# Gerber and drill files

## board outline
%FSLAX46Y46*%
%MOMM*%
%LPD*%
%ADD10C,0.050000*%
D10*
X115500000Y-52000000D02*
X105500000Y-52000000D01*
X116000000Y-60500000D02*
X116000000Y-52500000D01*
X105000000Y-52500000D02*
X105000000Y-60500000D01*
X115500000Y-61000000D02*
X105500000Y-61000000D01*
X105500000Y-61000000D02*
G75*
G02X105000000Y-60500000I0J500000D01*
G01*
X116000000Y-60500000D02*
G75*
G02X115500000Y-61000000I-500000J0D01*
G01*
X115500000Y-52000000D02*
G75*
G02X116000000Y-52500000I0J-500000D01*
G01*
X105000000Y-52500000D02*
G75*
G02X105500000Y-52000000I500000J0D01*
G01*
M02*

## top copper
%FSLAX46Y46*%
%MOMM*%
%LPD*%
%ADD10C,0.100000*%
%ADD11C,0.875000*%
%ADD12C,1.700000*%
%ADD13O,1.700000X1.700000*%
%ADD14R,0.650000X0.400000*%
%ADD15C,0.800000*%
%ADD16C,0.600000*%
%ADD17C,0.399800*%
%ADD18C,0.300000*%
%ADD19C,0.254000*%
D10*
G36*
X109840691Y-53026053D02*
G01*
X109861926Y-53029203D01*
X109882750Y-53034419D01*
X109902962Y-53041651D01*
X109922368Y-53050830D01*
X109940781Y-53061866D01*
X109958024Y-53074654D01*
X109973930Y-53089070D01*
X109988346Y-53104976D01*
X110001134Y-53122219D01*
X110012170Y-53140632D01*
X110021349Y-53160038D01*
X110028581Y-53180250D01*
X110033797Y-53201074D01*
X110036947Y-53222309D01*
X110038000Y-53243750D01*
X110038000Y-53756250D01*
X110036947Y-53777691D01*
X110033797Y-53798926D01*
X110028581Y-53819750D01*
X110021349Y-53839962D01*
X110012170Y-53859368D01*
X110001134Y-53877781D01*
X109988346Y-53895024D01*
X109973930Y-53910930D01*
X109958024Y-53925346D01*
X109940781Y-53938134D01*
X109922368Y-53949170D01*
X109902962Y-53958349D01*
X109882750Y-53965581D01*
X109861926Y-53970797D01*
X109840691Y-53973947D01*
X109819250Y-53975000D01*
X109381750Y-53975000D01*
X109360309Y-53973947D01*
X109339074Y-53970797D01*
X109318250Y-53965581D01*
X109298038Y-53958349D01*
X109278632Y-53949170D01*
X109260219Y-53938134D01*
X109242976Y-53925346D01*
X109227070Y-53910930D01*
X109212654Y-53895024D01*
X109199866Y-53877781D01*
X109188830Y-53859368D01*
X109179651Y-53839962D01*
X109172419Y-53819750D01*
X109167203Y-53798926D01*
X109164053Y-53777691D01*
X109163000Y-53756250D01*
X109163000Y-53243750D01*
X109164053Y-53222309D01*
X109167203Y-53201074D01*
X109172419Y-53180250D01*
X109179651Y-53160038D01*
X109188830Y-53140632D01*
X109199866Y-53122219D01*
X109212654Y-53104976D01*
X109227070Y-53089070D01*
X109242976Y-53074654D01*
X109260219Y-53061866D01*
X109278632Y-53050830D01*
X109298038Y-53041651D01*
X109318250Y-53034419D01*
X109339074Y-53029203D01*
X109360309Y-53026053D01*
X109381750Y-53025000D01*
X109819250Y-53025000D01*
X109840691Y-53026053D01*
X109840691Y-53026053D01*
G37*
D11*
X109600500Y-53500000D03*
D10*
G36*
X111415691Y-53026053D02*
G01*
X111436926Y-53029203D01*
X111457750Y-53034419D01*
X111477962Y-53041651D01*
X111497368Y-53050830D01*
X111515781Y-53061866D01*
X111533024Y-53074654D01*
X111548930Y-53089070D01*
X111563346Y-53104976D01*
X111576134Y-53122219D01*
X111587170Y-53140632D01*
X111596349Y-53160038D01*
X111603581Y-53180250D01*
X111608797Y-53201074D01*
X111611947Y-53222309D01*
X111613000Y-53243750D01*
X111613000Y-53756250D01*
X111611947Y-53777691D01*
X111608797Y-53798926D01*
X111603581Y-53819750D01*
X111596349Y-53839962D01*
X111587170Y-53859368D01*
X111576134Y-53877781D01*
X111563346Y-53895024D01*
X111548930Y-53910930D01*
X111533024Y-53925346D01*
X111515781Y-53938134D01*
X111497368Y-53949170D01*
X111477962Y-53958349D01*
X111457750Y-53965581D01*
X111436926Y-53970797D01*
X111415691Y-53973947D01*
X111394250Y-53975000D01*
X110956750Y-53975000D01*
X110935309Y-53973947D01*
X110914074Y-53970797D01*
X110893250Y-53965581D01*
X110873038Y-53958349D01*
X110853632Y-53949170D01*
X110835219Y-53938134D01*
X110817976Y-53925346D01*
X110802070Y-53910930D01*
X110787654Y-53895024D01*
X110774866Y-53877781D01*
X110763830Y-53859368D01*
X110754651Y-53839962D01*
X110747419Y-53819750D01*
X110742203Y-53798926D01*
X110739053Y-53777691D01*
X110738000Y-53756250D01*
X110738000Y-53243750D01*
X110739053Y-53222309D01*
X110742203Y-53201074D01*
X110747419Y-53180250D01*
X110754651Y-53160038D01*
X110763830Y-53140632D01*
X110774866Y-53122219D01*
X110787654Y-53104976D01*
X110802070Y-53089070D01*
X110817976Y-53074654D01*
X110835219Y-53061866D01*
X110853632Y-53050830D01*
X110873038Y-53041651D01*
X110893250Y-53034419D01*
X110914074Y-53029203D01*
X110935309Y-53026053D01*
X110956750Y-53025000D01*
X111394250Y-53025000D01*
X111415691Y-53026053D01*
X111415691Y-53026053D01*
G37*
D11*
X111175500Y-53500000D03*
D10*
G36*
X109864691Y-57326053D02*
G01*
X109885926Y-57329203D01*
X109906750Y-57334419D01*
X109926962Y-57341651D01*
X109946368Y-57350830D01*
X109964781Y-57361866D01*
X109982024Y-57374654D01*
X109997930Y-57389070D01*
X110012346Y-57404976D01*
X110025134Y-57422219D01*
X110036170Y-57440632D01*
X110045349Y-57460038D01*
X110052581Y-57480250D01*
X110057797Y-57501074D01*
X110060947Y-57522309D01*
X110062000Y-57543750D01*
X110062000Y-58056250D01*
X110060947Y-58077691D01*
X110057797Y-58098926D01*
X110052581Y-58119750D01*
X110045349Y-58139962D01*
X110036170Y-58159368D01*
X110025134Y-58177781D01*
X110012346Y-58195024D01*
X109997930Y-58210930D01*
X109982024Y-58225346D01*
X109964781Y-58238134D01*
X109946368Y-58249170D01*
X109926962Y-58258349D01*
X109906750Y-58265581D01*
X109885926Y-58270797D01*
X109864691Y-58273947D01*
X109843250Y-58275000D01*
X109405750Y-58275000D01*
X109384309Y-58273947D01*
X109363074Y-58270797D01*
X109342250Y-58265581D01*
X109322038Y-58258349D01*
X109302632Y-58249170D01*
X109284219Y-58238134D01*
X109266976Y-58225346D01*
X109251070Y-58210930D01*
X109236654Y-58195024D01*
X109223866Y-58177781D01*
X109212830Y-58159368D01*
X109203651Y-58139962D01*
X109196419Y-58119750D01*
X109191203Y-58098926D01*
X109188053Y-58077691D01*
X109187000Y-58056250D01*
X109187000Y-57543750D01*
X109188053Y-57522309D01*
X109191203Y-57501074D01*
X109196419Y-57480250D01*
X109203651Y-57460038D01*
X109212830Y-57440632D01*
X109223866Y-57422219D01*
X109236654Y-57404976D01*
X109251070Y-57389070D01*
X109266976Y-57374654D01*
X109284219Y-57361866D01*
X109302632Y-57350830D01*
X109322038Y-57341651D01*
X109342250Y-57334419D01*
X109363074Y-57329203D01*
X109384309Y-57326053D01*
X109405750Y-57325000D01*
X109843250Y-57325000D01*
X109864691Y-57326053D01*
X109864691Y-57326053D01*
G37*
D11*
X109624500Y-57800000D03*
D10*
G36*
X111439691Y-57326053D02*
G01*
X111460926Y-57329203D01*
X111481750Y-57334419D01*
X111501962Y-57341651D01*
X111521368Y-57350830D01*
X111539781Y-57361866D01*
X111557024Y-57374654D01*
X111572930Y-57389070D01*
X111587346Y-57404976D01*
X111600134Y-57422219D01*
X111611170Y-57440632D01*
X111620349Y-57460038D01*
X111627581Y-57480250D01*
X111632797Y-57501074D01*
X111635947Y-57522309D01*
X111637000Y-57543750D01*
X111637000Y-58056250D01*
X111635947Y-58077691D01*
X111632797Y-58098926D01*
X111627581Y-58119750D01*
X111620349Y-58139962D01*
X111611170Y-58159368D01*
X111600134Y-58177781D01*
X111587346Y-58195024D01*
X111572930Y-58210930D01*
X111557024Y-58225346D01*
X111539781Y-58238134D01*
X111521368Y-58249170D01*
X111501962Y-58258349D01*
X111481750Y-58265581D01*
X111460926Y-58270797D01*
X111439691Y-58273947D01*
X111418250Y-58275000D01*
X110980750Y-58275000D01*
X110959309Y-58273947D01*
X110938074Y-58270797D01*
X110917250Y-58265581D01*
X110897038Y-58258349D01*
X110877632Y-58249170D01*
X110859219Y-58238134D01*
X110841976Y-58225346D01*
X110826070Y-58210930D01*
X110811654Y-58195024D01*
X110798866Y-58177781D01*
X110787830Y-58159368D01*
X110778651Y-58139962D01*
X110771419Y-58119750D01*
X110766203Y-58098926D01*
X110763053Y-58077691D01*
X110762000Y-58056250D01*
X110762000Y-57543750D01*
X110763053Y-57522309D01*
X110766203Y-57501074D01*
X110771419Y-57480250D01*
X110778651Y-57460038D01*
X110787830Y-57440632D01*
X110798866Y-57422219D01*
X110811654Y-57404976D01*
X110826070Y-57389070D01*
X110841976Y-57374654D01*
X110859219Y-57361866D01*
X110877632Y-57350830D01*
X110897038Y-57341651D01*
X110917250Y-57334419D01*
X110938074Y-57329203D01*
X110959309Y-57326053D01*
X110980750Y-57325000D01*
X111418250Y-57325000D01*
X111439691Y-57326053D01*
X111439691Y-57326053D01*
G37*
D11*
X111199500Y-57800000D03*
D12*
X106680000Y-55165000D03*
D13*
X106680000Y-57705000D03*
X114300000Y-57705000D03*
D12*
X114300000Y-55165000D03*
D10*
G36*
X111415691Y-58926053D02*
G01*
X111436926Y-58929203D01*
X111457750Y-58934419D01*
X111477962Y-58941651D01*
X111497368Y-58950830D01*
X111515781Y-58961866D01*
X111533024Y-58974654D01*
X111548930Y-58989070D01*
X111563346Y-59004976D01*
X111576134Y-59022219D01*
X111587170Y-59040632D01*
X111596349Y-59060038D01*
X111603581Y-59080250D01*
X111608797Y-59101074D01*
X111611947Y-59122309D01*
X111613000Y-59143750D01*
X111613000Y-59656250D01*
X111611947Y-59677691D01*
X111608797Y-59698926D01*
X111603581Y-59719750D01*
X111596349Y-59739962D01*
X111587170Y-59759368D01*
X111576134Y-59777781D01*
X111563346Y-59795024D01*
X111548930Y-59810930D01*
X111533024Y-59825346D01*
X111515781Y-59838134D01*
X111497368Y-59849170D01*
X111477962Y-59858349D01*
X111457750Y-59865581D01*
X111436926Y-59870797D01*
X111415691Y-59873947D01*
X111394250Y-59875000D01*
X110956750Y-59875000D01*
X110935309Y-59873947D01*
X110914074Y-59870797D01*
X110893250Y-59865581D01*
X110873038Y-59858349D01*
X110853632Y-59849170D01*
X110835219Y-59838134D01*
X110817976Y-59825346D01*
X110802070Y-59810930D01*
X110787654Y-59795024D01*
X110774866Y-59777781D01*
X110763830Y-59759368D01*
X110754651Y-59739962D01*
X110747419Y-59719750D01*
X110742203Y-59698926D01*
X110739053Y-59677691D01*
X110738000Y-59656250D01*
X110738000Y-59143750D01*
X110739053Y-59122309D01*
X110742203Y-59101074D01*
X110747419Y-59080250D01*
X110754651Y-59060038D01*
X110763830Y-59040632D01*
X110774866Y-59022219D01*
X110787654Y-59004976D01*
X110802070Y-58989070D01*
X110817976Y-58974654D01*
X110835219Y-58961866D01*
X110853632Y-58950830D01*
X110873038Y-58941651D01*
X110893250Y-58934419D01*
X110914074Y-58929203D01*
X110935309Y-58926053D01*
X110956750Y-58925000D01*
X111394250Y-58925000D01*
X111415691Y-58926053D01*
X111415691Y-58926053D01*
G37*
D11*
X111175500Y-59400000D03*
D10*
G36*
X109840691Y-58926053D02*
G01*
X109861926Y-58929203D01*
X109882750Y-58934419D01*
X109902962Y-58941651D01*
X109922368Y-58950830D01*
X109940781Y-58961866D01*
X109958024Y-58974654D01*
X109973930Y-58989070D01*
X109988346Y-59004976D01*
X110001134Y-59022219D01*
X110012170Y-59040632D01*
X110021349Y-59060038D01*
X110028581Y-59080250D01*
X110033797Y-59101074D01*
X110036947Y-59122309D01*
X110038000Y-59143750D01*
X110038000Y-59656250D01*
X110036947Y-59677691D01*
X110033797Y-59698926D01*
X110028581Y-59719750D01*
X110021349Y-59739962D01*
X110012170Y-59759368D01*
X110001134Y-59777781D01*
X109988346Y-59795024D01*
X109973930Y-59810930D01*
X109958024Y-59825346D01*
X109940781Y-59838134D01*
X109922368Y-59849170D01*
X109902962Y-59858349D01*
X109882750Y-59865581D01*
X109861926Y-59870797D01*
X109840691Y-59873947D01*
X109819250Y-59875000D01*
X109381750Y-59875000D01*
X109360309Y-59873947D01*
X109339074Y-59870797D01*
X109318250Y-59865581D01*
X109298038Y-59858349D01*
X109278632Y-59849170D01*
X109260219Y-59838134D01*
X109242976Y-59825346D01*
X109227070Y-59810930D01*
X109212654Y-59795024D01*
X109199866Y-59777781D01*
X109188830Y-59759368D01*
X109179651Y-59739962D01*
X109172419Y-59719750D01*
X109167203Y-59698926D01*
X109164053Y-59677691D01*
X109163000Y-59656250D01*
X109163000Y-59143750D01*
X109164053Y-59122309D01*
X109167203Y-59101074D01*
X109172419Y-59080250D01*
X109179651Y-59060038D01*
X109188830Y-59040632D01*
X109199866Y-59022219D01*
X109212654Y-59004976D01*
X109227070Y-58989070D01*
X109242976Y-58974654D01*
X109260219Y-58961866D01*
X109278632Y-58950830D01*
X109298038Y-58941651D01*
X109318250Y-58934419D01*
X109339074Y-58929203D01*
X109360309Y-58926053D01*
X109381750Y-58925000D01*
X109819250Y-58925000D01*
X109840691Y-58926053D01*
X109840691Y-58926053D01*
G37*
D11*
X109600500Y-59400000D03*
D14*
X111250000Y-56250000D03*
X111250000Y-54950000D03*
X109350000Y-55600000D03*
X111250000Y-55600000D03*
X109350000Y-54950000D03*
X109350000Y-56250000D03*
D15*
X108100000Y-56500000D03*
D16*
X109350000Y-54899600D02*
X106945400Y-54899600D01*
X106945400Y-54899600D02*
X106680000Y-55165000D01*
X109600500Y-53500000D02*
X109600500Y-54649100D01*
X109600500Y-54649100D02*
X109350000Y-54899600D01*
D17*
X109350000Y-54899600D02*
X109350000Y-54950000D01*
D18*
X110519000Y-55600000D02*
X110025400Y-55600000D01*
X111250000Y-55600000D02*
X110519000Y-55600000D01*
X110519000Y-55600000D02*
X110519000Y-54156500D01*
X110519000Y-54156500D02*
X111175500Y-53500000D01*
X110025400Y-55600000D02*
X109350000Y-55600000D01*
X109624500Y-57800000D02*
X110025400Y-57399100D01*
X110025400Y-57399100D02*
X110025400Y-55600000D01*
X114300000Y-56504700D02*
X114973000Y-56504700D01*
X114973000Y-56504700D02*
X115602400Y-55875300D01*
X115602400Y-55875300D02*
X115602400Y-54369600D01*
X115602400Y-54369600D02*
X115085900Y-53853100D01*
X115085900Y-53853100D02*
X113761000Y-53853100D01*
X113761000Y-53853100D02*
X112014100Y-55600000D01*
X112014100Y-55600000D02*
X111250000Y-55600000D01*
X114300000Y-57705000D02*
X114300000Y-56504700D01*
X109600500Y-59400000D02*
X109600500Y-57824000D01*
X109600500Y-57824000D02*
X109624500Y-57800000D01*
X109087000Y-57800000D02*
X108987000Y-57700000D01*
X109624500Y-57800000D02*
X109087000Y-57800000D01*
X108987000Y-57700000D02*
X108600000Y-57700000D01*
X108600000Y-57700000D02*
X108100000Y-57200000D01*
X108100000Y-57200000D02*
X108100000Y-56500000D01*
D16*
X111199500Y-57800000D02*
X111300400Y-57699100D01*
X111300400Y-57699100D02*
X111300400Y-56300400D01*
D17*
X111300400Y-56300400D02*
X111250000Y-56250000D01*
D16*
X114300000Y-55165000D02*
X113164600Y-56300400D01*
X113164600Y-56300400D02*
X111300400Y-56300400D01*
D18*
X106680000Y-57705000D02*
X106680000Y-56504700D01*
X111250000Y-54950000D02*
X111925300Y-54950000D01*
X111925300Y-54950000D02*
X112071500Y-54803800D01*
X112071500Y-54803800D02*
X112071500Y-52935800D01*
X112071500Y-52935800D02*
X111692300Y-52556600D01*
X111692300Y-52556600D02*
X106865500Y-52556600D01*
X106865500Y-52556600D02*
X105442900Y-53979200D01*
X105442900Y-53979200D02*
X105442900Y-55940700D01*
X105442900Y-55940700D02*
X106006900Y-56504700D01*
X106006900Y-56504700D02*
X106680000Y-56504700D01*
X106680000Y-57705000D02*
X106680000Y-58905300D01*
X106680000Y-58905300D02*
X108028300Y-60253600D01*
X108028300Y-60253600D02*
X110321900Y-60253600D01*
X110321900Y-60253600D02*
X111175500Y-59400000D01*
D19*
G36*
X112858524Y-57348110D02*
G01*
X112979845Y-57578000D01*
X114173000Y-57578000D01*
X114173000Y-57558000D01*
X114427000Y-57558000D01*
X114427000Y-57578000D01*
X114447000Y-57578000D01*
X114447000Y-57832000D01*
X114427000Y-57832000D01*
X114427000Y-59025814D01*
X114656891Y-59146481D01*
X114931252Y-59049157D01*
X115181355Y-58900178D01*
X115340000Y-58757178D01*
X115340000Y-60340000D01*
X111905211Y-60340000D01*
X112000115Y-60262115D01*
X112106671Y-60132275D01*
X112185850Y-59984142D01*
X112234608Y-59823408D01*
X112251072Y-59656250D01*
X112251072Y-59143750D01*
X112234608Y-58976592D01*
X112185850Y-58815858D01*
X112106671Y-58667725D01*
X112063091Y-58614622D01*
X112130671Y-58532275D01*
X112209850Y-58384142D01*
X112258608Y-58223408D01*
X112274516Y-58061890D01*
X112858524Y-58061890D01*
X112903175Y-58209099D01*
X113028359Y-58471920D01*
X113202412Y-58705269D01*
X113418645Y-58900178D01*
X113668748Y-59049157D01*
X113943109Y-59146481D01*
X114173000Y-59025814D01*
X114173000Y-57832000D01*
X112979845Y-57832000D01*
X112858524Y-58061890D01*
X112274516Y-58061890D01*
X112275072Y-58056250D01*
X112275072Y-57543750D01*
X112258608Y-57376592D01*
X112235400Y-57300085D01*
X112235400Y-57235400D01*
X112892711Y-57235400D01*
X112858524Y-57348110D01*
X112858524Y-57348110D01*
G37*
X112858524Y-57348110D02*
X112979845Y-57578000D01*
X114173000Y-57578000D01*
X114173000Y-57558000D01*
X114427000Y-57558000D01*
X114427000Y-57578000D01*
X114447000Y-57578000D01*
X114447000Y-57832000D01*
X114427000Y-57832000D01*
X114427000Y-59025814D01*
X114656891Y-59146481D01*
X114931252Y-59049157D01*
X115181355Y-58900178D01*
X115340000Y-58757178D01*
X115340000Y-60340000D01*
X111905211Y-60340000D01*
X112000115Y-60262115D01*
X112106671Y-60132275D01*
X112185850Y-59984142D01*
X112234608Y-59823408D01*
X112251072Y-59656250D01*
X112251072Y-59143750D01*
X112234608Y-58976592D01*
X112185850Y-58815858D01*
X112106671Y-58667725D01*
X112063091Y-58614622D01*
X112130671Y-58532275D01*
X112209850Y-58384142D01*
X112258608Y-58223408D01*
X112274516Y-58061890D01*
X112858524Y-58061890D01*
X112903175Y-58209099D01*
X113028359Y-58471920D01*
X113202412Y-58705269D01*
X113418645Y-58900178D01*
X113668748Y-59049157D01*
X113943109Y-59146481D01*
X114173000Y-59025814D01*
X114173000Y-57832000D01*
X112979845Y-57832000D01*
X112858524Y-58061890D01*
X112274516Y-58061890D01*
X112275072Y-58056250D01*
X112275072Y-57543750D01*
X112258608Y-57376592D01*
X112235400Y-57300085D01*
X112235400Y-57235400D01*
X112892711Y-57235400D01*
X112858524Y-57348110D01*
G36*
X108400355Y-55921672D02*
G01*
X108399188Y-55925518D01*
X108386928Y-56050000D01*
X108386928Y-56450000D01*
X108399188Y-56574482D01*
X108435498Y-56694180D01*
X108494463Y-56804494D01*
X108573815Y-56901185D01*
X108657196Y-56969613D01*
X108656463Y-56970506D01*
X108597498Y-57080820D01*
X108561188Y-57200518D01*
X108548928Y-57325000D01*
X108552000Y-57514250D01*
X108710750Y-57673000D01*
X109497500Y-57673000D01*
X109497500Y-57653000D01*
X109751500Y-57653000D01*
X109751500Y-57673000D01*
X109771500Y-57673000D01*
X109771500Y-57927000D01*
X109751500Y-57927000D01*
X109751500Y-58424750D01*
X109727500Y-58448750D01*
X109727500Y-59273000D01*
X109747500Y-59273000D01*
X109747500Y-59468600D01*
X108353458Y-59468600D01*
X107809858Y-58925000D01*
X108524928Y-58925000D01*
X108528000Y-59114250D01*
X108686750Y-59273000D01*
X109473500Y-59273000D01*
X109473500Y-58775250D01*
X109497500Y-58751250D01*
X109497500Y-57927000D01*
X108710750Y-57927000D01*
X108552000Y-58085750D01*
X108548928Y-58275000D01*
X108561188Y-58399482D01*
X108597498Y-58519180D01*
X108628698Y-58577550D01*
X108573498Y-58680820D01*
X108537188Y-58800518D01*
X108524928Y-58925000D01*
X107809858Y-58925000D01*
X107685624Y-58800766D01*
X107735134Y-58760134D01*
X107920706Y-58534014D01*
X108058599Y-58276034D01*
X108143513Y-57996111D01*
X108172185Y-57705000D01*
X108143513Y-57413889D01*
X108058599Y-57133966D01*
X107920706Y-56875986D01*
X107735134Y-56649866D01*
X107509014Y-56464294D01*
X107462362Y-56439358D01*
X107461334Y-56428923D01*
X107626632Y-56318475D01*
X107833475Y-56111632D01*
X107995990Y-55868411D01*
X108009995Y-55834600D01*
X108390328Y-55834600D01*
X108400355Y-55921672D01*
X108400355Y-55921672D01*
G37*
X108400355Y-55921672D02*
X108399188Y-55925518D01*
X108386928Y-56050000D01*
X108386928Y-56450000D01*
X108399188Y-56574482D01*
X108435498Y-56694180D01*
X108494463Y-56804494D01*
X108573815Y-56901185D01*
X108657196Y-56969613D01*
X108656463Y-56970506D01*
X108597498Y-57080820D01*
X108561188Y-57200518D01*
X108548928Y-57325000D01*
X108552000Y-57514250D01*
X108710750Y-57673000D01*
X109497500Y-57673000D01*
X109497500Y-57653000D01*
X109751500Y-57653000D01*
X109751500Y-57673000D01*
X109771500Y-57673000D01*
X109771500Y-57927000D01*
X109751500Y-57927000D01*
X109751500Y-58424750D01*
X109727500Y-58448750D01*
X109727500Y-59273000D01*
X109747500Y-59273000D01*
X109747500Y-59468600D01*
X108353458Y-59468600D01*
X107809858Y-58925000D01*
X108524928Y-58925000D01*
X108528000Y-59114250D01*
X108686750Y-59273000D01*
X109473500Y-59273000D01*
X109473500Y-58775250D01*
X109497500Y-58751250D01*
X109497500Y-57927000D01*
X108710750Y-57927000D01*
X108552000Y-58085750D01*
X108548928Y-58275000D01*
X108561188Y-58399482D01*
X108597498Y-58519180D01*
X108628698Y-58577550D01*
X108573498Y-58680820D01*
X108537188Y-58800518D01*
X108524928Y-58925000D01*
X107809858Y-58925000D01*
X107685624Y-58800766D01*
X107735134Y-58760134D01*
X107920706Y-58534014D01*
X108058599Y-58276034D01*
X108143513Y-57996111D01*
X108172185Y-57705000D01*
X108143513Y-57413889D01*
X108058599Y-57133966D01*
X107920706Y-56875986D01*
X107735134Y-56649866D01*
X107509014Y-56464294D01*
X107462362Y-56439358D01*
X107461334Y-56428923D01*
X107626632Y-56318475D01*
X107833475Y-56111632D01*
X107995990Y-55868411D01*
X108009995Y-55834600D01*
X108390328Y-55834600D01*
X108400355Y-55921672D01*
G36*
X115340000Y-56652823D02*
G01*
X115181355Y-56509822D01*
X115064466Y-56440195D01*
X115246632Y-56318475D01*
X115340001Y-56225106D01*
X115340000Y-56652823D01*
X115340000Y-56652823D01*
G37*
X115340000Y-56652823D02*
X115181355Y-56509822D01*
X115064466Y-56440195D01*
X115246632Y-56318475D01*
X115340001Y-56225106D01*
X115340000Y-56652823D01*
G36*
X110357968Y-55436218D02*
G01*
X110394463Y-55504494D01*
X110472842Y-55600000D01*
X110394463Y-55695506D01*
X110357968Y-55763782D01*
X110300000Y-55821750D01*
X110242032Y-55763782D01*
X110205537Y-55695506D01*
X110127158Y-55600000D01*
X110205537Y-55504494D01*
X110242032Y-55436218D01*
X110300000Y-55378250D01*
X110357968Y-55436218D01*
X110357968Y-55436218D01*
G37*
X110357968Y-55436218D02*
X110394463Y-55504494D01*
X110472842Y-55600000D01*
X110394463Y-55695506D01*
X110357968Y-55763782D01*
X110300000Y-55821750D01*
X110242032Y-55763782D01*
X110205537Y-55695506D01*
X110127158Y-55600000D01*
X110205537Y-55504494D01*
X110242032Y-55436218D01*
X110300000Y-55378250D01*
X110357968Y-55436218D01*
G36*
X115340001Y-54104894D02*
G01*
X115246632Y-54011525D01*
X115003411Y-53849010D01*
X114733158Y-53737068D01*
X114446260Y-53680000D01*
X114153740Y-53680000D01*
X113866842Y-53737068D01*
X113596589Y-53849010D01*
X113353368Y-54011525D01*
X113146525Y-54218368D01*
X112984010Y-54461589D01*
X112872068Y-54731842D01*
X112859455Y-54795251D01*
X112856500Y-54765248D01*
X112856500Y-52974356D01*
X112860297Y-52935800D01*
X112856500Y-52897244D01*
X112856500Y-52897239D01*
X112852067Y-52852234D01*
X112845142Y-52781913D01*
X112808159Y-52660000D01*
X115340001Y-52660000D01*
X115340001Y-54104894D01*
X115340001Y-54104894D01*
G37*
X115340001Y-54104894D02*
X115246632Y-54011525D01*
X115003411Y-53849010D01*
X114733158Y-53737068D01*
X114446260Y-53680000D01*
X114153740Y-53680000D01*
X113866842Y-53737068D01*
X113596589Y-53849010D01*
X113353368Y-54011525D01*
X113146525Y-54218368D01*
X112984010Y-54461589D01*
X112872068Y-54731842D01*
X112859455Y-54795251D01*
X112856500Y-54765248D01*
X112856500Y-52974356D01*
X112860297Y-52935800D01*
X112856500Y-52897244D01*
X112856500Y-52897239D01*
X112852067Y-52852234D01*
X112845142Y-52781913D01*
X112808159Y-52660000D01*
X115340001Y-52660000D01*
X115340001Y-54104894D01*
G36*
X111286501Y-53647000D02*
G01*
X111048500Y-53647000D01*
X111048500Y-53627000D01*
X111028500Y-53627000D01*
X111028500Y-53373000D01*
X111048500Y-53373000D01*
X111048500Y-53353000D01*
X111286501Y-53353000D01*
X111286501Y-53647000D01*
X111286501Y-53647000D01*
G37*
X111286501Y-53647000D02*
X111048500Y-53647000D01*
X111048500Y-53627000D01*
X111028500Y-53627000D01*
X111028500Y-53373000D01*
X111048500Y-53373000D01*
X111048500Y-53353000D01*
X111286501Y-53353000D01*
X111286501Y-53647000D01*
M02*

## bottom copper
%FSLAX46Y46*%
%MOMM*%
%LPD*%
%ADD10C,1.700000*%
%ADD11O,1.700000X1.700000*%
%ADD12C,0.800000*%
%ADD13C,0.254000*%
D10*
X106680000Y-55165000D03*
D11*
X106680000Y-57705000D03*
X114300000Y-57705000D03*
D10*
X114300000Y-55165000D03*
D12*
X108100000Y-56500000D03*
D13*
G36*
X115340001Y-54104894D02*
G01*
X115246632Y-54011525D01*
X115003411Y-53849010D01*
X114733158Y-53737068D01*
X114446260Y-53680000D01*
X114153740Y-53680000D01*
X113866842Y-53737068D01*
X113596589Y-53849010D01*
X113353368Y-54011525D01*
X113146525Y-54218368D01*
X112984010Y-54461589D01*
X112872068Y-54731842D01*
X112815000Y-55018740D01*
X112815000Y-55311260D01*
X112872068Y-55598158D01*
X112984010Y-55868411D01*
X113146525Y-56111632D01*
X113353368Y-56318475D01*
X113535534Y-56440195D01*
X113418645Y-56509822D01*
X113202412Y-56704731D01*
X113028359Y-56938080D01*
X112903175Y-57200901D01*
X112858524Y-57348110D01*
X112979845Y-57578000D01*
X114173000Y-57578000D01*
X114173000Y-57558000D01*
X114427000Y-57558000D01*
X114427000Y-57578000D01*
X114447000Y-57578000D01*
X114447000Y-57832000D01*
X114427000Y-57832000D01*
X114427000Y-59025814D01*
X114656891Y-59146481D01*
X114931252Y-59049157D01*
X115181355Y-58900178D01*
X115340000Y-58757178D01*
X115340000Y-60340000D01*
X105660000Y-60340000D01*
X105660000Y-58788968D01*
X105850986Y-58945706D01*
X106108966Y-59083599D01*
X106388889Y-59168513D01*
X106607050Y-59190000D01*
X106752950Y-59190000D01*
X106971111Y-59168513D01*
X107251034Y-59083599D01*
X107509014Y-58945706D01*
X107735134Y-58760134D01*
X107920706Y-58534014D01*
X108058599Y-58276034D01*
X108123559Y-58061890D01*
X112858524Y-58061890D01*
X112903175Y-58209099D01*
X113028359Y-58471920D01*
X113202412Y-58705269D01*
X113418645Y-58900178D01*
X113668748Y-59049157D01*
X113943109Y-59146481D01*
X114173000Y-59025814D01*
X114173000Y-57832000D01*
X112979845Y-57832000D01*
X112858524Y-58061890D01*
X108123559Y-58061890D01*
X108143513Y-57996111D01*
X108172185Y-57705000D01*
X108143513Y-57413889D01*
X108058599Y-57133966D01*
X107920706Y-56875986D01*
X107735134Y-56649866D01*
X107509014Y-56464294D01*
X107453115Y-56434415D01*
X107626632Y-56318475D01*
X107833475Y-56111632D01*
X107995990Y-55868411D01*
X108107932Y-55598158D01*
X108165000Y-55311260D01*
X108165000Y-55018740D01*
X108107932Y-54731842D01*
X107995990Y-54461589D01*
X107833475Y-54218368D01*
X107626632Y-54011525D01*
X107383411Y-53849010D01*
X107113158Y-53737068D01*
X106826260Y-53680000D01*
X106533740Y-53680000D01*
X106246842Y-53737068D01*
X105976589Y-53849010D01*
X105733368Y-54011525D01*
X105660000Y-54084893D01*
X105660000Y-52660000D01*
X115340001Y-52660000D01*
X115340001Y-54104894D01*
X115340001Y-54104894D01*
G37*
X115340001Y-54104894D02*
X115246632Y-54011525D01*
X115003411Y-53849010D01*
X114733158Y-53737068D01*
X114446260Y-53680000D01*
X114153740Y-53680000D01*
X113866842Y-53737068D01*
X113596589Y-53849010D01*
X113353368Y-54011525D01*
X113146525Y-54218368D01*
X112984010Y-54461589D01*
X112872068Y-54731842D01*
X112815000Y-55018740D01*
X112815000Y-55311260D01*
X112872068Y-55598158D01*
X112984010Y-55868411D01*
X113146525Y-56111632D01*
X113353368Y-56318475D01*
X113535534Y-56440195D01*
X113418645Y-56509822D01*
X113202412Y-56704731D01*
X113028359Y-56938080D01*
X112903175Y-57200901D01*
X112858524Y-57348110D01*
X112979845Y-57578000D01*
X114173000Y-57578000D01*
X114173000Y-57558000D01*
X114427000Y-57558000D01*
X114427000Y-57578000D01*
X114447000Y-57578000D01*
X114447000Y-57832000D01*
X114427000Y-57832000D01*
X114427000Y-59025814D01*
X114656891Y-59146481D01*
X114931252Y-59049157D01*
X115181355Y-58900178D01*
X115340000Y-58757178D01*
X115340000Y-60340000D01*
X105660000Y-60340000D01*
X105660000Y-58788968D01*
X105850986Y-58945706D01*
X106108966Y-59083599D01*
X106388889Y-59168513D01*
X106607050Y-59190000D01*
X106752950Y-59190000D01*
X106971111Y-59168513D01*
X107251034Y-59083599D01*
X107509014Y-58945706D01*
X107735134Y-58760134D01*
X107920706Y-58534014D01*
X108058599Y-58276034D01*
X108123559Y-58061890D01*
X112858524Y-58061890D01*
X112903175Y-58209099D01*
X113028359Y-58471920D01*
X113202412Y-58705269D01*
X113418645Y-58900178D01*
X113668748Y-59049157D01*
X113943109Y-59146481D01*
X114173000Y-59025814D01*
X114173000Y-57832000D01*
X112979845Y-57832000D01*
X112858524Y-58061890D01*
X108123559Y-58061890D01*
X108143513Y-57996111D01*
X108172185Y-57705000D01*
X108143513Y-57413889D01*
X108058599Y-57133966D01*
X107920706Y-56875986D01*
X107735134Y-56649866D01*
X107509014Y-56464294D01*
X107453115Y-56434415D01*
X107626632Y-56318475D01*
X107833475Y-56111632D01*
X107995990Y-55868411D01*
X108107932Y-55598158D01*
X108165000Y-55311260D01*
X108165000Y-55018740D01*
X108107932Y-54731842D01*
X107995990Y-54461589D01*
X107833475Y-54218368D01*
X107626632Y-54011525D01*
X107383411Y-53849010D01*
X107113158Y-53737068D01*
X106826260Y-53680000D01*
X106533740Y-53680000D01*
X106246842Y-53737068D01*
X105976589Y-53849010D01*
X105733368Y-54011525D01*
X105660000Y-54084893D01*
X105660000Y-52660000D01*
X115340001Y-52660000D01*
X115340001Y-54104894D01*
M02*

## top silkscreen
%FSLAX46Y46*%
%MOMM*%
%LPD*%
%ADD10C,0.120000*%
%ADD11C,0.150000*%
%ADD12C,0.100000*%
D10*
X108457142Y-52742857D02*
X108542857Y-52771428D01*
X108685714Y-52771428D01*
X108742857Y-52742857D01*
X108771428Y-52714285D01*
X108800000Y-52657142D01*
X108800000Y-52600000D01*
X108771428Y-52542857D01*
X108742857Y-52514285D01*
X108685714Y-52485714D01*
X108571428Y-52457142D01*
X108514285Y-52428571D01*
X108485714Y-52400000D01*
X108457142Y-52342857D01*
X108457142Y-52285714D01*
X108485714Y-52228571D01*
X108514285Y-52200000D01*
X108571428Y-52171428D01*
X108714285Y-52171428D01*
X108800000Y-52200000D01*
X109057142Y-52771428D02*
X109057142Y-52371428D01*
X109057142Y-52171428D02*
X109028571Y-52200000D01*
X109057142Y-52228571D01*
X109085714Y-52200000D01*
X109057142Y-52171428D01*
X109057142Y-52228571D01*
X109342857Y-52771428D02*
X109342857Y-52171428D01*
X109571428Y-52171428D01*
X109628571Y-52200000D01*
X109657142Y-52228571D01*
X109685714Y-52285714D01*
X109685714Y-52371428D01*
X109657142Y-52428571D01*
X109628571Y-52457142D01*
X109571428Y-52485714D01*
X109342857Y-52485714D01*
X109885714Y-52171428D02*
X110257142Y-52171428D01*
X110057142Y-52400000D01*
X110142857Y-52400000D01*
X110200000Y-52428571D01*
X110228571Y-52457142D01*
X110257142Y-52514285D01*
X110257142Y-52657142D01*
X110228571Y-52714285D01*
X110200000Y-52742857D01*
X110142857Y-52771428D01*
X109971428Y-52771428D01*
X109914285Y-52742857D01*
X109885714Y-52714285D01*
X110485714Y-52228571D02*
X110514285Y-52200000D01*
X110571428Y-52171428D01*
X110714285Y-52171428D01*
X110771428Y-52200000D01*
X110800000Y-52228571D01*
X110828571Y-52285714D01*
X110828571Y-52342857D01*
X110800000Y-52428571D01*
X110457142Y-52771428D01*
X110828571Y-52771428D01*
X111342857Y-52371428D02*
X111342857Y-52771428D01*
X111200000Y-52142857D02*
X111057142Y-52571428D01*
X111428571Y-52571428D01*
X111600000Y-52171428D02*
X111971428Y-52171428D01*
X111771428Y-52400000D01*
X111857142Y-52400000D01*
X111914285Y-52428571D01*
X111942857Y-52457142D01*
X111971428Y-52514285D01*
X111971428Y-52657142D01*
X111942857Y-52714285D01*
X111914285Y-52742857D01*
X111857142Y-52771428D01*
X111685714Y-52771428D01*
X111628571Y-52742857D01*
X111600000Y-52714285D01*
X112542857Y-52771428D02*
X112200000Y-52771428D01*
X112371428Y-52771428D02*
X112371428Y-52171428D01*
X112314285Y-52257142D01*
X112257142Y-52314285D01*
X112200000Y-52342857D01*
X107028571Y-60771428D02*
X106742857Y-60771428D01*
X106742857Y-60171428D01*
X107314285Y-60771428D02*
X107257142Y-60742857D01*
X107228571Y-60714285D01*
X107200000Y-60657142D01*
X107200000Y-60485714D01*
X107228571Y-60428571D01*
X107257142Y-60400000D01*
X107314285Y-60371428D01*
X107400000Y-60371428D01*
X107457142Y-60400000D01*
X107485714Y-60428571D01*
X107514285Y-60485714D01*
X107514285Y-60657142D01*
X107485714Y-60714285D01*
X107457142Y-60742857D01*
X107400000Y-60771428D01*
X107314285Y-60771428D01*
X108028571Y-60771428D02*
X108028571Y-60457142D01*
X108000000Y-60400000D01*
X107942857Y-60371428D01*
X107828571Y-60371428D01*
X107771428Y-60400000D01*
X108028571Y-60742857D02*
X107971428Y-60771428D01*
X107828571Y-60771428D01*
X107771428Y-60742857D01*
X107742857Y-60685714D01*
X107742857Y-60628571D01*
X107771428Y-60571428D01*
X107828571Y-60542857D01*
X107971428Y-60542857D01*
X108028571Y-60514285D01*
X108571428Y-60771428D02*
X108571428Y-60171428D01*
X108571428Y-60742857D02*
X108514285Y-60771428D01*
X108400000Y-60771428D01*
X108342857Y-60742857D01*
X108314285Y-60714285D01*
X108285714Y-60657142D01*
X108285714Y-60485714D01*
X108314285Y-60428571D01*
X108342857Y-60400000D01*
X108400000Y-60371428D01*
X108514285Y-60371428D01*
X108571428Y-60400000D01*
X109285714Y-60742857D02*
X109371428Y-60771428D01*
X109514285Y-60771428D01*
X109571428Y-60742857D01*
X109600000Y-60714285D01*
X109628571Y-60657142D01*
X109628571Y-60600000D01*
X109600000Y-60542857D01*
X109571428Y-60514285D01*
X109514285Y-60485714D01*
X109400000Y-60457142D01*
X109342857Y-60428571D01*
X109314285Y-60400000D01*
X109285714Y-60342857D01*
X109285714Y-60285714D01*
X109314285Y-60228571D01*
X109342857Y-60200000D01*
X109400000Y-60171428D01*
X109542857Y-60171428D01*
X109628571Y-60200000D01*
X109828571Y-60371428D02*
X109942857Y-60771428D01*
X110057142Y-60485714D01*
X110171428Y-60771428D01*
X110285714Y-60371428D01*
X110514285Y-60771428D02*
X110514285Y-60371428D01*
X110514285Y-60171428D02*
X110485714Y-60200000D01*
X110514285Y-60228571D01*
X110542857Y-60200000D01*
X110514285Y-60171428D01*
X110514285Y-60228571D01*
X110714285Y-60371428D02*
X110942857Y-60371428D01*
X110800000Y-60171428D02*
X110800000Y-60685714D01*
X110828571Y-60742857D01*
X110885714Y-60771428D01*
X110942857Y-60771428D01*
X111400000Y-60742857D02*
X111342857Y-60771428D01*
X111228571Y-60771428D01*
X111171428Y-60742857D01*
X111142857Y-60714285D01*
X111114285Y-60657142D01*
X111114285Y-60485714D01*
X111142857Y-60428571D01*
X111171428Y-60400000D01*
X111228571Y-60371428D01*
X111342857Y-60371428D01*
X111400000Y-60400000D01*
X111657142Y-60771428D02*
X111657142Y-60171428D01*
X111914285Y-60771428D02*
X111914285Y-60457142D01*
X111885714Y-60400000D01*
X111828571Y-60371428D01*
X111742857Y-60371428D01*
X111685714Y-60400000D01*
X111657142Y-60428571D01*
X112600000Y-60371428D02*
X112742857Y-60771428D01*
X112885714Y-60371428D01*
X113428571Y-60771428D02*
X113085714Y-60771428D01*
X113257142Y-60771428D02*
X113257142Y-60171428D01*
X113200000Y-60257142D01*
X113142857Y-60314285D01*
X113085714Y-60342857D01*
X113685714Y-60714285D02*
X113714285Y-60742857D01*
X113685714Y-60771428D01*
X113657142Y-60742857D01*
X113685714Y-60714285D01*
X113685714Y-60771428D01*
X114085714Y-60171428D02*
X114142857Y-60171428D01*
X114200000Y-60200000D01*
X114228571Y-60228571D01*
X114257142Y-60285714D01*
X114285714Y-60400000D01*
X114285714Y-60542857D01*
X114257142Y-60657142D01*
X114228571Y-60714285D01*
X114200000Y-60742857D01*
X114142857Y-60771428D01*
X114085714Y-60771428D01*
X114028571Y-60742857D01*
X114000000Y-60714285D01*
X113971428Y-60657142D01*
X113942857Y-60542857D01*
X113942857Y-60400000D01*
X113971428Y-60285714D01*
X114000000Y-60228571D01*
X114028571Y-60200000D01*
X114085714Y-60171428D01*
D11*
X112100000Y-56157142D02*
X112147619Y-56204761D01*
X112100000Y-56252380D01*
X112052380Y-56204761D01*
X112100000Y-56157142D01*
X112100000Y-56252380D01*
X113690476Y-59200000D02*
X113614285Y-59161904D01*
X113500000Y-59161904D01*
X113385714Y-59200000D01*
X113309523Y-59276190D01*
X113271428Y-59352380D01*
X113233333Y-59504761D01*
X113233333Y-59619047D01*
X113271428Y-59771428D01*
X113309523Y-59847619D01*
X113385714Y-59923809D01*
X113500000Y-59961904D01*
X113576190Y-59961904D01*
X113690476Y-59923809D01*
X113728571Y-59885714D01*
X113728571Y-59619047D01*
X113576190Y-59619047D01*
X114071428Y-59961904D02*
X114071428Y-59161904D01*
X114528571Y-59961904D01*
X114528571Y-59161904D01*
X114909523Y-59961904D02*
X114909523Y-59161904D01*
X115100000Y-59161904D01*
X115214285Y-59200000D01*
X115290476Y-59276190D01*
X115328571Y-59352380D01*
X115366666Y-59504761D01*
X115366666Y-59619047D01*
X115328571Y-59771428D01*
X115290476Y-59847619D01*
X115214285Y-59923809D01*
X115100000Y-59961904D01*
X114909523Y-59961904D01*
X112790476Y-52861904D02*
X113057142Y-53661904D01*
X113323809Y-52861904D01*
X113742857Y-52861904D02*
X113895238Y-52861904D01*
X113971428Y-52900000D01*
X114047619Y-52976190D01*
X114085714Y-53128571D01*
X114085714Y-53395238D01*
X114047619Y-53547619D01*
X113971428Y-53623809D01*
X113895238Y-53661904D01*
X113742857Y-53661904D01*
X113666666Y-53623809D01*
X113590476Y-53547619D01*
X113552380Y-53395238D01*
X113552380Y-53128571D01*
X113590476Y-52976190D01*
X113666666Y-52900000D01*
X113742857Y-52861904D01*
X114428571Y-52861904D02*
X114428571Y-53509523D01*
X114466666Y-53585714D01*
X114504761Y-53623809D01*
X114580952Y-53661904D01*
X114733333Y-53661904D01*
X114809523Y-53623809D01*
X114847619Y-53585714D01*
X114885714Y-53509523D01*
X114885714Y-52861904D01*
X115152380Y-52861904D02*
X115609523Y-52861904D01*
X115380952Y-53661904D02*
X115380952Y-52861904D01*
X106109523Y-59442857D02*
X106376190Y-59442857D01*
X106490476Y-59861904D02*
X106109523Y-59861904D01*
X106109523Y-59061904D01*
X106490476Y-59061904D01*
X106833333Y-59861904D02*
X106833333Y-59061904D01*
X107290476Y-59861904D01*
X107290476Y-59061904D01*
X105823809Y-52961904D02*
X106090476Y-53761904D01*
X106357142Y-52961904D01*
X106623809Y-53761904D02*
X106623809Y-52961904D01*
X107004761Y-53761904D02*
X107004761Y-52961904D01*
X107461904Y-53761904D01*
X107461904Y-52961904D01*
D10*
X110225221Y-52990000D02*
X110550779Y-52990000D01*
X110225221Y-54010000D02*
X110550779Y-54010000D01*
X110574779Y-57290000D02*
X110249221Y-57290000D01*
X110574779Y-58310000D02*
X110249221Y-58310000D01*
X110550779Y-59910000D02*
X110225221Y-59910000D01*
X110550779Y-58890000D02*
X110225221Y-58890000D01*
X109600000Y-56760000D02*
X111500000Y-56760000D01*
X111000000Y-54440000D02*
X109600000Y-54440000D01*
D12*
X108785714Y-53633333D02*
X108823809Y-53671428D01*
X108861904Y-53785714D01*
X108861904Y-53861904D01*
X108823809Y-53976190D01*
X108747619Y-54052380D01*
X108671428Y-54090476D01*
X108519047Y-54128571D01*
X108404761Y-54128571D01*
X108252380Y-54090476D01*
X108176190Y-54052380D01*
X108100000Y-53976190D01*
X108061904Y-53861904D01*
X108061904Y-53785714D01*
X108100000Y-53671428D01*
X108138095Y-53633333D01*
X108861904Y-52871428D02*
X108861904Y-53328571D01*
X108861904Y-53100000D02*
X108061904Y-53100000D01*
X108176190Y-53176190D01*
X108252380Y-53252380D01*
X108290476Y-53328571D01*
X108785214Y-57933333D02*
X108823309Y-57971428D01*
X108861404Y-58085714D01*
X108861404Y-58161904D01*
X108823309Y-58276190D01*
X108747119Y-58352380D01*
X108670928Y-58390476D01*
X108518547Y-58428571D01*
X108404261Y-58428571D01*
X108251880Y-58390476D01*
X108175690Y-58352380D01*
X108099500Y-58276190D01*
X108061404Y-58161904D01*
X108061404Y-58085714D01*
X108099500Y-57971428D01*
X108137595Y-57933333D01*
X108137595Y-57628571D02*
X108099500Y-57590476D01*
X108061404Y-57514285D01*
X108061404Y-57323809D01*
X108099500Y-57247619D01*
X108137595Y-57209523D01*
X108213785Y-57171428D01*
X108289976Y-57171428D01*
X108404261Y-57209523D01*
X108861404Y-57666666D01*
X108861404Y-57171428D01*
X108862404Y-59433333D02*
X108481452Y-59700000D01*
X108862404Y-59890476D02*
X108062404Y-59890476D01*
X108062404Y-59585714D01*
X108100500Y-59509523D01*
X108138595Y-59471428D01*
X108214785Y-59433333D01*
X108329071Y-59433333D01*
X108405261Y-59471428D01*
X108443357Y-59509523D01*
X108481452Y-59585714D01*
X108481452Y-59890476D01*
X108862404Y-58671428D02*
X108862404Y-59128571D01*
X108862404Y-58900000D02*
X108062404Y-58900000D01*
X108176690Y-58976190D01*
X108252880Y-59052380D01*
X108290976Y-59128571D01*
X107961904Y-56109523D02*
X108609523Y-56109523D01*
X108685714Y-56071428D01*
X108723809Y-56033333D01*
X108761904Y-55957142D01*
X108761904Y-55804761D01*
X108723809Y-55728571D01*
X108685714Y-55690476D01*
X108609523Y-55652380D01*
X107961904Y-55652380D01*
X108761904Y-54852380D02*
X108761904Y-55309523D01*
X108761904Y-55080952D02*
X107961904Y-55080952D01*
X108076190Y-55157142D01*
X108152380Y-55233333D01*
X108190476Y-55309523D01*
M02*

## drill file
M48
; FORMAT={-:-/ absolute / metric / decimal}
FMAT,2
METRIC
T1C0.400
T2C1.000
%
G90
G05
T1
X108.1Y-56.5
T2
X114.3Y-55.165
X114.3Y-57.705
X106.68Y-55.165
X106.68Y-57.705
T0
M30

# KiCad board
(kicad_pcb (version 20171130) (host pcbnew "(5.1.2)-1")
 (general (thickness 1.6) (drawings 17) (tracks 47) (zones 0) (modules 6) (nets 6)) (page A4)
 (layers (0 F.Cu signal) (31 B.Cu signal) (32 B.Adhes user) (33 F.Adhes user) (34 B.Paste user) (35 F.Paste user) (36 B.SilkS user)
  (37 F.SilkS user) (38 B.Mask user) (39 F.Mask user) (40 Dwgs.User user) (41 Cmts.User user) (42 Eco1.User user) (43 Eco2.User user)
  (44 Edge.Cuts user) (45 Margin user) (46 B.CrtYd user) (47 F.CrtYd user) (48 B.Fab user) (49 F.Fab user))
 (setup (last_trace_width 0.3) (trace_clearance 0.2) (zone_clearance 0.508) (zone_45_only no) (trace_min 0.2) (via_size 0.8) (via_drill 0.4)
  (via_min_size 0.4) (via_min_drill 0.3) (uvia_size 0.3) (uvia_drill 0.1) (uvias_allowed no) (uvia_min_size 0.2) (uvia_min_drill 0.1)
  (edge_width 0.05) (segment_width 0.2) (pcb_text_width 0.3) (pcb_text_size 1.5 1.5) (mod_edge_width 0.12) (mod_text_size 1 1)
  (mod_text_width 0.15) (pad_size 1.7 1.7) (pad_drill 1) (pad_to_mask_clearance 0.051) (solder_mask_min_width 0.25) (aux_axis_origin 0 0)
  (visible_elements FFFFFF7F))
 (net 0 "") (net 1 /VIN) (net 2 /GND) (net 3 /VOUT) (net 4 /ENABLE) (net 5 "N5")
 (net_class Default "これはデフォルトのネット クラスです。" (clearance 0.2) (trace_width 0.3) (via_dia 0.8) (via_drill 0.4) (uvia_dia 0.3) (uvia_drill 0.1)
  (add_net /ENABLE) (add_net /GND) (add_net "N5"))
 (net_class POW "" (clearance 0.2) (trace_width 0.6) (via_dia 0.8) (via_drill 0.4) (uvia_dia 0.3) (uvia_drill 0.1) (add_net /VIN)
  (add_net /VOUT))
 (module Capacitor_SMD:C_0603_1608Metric (layer F.Cu) (at 110.388 53.5)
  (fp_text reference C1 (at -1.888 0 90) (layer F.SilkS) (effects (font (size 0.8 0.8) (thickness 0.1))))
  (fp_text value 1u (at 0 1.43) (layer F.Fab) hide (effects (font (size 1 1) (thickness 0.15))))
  (fp_line (start -0.162779 -0.51) (end 0.162779 -0.51) (layer F.SilkS) (width 0.12))
  (fp_line (start -0.162779 0.51) (end 0.162779 0.51) (layer F.SilkS) (width 0.12))
  (pad 1 smd roundrect (at -0.7875 0) (size 0.875 0.95) (layers F.Cu F.Paste F.Mask) (roundrect_rratio 0.25) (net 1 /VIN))
  (pad 2 smd roundrect (at 0.7875 0) (size 0.875 0.95) (layers F.Cu F.Paste F.Mask) (roundrect_rratio 0.25) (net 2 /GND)))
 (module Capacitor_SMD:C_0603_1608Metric (layer F.Cu) (at 110.412 57.8 180)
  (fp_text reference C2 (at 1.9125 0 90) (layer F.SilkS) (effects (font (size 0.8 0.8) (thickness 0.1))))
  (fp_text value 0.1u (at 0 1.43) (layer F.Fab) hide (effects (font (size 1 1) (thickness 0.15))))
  (fp_line (start -0.162779 0.51) (end 0.162779 0.51) (layer F.SilkS) (width 0.12))
  (fp_line (start -0.162779 -0.51) (end 0.162779 -0.51) (layer F.SilkS) (width 0.12))
  (pad 2 smd roundrect (at 0.7875 0 180) (size 0.875 0.95) (layers F.Cu F.Paste F.Mask) (roundrect_rratio 0.25) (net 2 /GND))
  (pad 1 smd roundrect (at -0.7875 0 180) (size 0.875 0.95) (layers F.Cu F.Paste F.Mask) (roundrect_rratio 0.25) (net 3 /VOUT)))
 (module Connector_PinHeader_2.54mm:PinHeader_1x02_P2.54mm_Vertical (layer B.Cu) (at 106.68 55.165 180)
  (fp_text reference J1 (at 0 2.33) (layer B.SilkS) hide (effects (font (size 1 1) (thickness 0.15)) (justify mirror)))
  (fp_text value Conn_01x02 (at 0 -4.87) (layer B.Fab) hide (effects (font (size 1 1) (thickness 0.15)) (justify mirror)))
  (pad 1 thru_hole circle (at 0 0 180) (size 1.7 1.7) (drill 1) (layers *.Cu *.Mask) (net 1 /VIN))
  (pad 2 thru_hole oval (at 0 -2.54 180) (size 1.7 1.7) (drill 1) (layers *.Cu *.Mask) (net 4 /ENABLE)))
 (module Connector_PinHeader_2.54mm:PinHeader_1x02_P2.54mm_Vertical (layer B.Cu) (at 114.3 55.165 180)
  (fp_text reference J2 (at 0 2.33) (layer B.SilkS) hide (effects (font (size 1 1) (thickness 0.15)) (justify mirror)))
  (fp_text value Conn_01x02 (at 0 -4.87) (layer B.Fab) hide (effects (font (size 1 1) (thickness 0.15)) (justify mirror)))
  (pad 2 thru_hole oval (at 0 -2.54 180) (size 1.7 1.7) (drill 1) (layers *.Cu *.Mask) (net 2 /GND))
  (pad 1 thru_hole circle (at 0 0 180) (size 1.7 1.7) (drill 1) (layers *.Cu *.Mask) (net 3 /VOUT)))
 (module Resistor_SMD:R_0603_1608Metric (layer F.Cu) (at 110.388 59.4 180)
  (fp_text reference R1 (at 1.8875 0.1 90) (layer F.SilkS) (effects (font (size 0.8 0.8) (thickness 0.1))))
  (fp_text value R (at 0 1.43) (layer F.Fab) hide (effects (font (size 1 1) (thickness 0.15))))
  (fp_line (start -0.162779 -0.51) (end 0.162779 -0.51) (layer F.SilkS) (width 0.12))
  (fp_line (start -0.162779 0.51) (end 0.162779 0.51) (layer F.SilkS) (width 0.12))
  (pad 1 smd roundrect (at -0.7875 0 180) (size 0.875 0.95) (layers F.Cu F.Paste F.Mask) (roundrect_rratio 0.25) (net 4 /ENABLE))
  (pad 2 smd roundrect (at 0.7875 0 180) (size 0.875 0.95) (layers F.Cu F.Paste F.Mask) (roundrect_rratio 0.25) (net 2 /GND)))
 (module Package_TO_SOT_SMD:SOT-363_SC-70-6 (layer F.Cu) (at 110.3 55.6 180)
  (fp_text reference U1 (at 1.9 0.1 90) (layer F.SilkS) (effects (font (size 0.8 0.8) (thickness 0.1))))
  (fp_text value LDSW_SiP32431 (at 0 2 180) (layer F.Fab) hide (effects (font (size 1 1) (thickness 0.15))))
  (fp_line (start 0.7 -1.16) (end -1.2 -1.16) (layer F.SilkS) (width 0.12))
  (fp_line (start -0.7 1.16) (end 0.7 1.16) (layer F.SilkS) (width 0.12))
  (pad 1 smd rect (at -0.95 -0.65 180) (size 0.65 0.4) (layers F.Cu F.Paste F.Mask) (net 3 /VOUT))
  (pad 3 smd rect (at -0.95 0.65 180) (size 0.65 0.4) (layers F.Cu F.Paste F.Mask) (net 4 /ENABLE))
  (pad 5 smd rect (at 0.95 0 180) (size 0.65 0.4) (layers F.Cu F.Paste F.Mask) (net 2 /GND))
  (pad 2 smd rect (at -0.95 0 180) (size 0.65 0.4) (layers F.Cu F.Paste F.Mask) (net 2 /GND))
  (pad 4 smd rect (at 0.95 0.65 180) (size 0.65 0.4) (layers F.Cu F.Paste F.Mask) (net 1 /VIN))
  (pad 6 smd rect (at 0.95 -0.65 180) (size 0.65 0.4) (layers F.Cu F.Paste F.Mask) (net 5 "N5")))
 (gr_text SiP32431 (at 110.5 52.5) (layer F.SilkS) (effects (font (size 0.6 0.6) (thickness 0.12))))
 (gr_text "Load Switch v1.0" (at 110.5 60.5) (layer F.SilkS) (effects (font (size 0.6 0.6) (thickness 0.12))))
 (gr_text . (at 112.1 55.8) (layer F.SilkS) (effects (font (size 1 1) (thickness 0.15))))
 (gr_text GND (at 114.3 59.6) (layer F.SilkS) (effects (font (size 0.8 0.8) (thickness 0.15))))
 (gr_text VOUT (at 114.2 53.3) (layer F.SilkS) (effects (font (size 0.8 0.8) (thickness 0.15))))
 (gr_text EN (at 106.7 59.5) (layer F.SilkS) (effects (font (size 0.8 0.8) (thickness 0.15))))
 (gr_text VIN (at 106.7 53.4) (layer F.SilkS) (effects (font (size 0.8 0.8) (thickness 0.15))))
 (gr_line (start 115.5 52) (end 105.5 52) (layer Edge.Cuts) (width 0.05))
 (gr_line (start 116 60.5) (end 116 52.5) (layer Edge.Cuts) (width 0.05))
 (gr_line (start 105 52.5) (end 105 60.5) (layer Edge.Cuts) (width 0.05))
 (gr_line (start 115.5 61) (end 105.5 61) (layer Edge.Cuts) (width 0.05))
 (gr_arc (start 105.5 60.5) (end 105 60.5) (angle -90) (layer Edge.Cuts) (width 0.05))
 (gr_arc (start 115.5 60.5) (end 115.5 61) (angle -90) (layer Edge.Cuts) (width 0.05))
 (gr_arc (start 115.5 52.5) (end 116 52.5) (angle -90) (layer Edge.Cuts) (width 0.05))
 (gr_arc (start 105.5 52.5) (end 105.5 52) (angle -90) (layer Edge.Cuts) (width 0.05))
 (segment (start 109.35 54.8996) (end 106.9454 54.8996) (width 0.6) (layer F.Cu) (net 1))
 (segment (start 106.9454 54.8996) (end 106.68 55.165) (width 0.6) (layer F.Cu) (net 1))
 (segment (start 109.6005 53.5) (end 109.6005 54.6491) (width 0.6) (layer F.Cu) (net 1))
 (segment (start 109.6005 54.6491) (end 109.35 54.8996) (width 0.6) (layer F.Cu) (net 1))
 (segment (start 109.35 54.8996) (end 109.35 54.95) (width 0.3998) (layer F.Cu) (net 1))
 (segment (start 110.519 55.6) (end 110.0254 55.6) (width 0.3) (layer F.Cu) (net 2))
 (segment (start 111.25 55.6) (end 110.519 55.6) (width 0.3) (layer F.Cu) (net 2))
 (segment (start 110.519 55.6) (end 110.519 54.1565) (width 0.3) (layer F.Cu) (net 2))
 (segment (start 110.519 54.1565) (end 111.1755 53.5) (width 0.3) (layer F.Cu) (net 2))
 (segment (start 110.0254 55.6) (end 109.35 55.6) (width 0.3) (layer F.Cu) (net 2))
 (segment (start 109.6245 57.8) (end 110.0254 57.3991) (width 0.3) (layer F.Cu) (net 2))
 (segment (start 110.0254 57.3991) (end 110.0254 55.6) (width 0.3) (layer F.Cu) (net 2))
 (segment (start 114.3 56.5047) (end 114.973 56.5047) (width 0.3) (layer F.Cu) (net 2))
 (segment (start 114.973 56.5047) (end 115.6024 55.8753) (width 0.3) (layer F.Cu) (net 2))
 (segment (start 115.6024 55.8753) (end 115.6024 54.3696) (width 0.3) (layer F.Cu) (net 2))
 (segment (start 115.6024 54.3696) (end 115.0859 53.8531) (width 0.3) (layer F.Cu) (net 2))
 (segment (start 115.0859 53.8531) (end 113.761 53.8531) (width 0.3) (layer F.Cu) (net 2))
 (segment (start 113.761 53.8531) (end 112.0141 55.6) (width 0.3) (layer F.Cu) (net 2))
 (segment (start 112.0141 55.6) (end 111.25 55.6) (width 0.3) (layer F.Cu) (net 2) (status 800000))
 (segment (start 114.3 57.705) (end 114.3 56.5047) (width 0.3) (layer F.Cu) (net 2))
 (segment (start 109.6005 59.4) (end 109.6005 57.824) (width 0.3) (layer F.Cu) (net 2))
 (segment (start 109.6005 57.824) (end 109.6245 57.8) (width 0.3) (layer F.Cu) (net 2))
 (segment (start 109.087 57.8) (end 108.987 57.7) (width 0.3) (layer F.Cu) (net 2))
 (segment (start 109.6245 57.8) (end 109.087 57.8) (width 0.3) (layer F.Cu) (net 2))
 (segment (start 108.987 57.7) (end 108.6 57.7) (width 0.3) (layer F.Cu) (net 2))
 (via (at 108.1 56.5) (size 0.8) (drill 0.4) (layers F.Cu B.Cu) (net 2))
 (segment (start 108.6 57.7) (end 108.1 57.2) (width 0.3) (layer F.Cu) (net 2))
 (segment (start 108.1 57.2) (end 108.1 56.5) (width 0.3) (layer F.Cu) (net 2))
 (segment (start 111.1995 57.8) (end 111.3004 57.6991) (width 0.6) (layer F.Cu) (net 3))
 (segment (start 111.3004 57.6991) (end 111.3004 56.3004) (width 0.6) (layer F.Cu) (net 3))
 (segment (start 111.3004 56.3004) (end 111.25 56.25) (width 0.3998) (layer F.Cu) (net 3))
 (segment (start 114.3 55.165) (end 113.1646 56.3004) (width 0.6) (layer F.Cu) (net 3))
 (segment (start 113.1646 56.3004) (end 111.3004 56.3004) (width 0.6) (layer F.Cu) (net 3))
 (segment (start 106.68 57.705) (end 106.68 56.5047) (width 0.3) (layer F.Cu) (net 4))
 (segment (start 111.25 54.95) (end 111.9253 54.95) (width 0.3) (layer F.Cu) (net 4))
 (segment (start 111.9253 54.95) (end 112.0715 54.8038) (width 0.3) (layer F.Cu) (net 4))
 (segment (start 112.0715 54.8038) (end 112.0715 52.9358) (width 0.3) (layer F.Cu) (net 4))
 (segment (start 112.0715 52.9358) (end 111.6923 52.5566) (width 0.3) (layer F.Cu) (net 4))
 (segment (start 111.6923 52.5566) (end 106.8655 52.5566) (width 0.3) (layer F.Cu) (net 4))
 (segment (start 106.8655 52.5566) (end 105.4429 53.9792) (width 0.3) (layer F.Cu) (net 4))
 (segment (start 105.4429 53.9792) (end 105.4429 55.9407) (width 0.3) (layer F.Cu) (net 4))
 (segment (start 105.4429 55.9407) (end 106.0069 56.5047) (width 0.3) (layer F.Cu) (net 4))
 (segment (start 106.0069 56.5047) (end 106.68 56.5047) (width 0.3) (layer F.Cu) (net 4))
 (segment (start 106.68 57.705) (end 106.68 58.9053) (width 0.3) (layer F.Cu) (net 4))
 (segment (start 106.68 58.9053) (end 108.0283 60.2536) (width 0.3) (layer F.Cu) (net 4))
 (segment (start 108.0283 60.2536) (end 110.3219 60.2536) (width 0.3) (layer F.Cu) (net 4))
 (segment (start 110.3219 60.2536) (end 111.1755 59.4) (width 0.3) (layer F.Cu) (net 4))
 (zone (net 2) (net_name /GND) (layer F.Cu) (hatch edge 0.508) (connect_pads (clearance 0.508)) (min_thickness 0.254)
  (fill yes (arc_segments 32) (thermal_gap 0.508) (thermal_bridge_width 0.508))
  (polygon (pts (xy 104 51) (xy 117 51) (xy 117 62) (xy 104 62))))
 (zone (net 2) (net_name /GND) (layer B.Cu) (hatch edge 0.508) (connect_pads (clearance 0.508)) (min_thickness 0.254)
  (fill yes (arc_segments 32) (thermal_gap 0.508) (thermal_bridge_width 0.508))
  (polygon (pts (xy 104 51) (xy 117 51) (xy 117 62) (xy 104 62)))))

